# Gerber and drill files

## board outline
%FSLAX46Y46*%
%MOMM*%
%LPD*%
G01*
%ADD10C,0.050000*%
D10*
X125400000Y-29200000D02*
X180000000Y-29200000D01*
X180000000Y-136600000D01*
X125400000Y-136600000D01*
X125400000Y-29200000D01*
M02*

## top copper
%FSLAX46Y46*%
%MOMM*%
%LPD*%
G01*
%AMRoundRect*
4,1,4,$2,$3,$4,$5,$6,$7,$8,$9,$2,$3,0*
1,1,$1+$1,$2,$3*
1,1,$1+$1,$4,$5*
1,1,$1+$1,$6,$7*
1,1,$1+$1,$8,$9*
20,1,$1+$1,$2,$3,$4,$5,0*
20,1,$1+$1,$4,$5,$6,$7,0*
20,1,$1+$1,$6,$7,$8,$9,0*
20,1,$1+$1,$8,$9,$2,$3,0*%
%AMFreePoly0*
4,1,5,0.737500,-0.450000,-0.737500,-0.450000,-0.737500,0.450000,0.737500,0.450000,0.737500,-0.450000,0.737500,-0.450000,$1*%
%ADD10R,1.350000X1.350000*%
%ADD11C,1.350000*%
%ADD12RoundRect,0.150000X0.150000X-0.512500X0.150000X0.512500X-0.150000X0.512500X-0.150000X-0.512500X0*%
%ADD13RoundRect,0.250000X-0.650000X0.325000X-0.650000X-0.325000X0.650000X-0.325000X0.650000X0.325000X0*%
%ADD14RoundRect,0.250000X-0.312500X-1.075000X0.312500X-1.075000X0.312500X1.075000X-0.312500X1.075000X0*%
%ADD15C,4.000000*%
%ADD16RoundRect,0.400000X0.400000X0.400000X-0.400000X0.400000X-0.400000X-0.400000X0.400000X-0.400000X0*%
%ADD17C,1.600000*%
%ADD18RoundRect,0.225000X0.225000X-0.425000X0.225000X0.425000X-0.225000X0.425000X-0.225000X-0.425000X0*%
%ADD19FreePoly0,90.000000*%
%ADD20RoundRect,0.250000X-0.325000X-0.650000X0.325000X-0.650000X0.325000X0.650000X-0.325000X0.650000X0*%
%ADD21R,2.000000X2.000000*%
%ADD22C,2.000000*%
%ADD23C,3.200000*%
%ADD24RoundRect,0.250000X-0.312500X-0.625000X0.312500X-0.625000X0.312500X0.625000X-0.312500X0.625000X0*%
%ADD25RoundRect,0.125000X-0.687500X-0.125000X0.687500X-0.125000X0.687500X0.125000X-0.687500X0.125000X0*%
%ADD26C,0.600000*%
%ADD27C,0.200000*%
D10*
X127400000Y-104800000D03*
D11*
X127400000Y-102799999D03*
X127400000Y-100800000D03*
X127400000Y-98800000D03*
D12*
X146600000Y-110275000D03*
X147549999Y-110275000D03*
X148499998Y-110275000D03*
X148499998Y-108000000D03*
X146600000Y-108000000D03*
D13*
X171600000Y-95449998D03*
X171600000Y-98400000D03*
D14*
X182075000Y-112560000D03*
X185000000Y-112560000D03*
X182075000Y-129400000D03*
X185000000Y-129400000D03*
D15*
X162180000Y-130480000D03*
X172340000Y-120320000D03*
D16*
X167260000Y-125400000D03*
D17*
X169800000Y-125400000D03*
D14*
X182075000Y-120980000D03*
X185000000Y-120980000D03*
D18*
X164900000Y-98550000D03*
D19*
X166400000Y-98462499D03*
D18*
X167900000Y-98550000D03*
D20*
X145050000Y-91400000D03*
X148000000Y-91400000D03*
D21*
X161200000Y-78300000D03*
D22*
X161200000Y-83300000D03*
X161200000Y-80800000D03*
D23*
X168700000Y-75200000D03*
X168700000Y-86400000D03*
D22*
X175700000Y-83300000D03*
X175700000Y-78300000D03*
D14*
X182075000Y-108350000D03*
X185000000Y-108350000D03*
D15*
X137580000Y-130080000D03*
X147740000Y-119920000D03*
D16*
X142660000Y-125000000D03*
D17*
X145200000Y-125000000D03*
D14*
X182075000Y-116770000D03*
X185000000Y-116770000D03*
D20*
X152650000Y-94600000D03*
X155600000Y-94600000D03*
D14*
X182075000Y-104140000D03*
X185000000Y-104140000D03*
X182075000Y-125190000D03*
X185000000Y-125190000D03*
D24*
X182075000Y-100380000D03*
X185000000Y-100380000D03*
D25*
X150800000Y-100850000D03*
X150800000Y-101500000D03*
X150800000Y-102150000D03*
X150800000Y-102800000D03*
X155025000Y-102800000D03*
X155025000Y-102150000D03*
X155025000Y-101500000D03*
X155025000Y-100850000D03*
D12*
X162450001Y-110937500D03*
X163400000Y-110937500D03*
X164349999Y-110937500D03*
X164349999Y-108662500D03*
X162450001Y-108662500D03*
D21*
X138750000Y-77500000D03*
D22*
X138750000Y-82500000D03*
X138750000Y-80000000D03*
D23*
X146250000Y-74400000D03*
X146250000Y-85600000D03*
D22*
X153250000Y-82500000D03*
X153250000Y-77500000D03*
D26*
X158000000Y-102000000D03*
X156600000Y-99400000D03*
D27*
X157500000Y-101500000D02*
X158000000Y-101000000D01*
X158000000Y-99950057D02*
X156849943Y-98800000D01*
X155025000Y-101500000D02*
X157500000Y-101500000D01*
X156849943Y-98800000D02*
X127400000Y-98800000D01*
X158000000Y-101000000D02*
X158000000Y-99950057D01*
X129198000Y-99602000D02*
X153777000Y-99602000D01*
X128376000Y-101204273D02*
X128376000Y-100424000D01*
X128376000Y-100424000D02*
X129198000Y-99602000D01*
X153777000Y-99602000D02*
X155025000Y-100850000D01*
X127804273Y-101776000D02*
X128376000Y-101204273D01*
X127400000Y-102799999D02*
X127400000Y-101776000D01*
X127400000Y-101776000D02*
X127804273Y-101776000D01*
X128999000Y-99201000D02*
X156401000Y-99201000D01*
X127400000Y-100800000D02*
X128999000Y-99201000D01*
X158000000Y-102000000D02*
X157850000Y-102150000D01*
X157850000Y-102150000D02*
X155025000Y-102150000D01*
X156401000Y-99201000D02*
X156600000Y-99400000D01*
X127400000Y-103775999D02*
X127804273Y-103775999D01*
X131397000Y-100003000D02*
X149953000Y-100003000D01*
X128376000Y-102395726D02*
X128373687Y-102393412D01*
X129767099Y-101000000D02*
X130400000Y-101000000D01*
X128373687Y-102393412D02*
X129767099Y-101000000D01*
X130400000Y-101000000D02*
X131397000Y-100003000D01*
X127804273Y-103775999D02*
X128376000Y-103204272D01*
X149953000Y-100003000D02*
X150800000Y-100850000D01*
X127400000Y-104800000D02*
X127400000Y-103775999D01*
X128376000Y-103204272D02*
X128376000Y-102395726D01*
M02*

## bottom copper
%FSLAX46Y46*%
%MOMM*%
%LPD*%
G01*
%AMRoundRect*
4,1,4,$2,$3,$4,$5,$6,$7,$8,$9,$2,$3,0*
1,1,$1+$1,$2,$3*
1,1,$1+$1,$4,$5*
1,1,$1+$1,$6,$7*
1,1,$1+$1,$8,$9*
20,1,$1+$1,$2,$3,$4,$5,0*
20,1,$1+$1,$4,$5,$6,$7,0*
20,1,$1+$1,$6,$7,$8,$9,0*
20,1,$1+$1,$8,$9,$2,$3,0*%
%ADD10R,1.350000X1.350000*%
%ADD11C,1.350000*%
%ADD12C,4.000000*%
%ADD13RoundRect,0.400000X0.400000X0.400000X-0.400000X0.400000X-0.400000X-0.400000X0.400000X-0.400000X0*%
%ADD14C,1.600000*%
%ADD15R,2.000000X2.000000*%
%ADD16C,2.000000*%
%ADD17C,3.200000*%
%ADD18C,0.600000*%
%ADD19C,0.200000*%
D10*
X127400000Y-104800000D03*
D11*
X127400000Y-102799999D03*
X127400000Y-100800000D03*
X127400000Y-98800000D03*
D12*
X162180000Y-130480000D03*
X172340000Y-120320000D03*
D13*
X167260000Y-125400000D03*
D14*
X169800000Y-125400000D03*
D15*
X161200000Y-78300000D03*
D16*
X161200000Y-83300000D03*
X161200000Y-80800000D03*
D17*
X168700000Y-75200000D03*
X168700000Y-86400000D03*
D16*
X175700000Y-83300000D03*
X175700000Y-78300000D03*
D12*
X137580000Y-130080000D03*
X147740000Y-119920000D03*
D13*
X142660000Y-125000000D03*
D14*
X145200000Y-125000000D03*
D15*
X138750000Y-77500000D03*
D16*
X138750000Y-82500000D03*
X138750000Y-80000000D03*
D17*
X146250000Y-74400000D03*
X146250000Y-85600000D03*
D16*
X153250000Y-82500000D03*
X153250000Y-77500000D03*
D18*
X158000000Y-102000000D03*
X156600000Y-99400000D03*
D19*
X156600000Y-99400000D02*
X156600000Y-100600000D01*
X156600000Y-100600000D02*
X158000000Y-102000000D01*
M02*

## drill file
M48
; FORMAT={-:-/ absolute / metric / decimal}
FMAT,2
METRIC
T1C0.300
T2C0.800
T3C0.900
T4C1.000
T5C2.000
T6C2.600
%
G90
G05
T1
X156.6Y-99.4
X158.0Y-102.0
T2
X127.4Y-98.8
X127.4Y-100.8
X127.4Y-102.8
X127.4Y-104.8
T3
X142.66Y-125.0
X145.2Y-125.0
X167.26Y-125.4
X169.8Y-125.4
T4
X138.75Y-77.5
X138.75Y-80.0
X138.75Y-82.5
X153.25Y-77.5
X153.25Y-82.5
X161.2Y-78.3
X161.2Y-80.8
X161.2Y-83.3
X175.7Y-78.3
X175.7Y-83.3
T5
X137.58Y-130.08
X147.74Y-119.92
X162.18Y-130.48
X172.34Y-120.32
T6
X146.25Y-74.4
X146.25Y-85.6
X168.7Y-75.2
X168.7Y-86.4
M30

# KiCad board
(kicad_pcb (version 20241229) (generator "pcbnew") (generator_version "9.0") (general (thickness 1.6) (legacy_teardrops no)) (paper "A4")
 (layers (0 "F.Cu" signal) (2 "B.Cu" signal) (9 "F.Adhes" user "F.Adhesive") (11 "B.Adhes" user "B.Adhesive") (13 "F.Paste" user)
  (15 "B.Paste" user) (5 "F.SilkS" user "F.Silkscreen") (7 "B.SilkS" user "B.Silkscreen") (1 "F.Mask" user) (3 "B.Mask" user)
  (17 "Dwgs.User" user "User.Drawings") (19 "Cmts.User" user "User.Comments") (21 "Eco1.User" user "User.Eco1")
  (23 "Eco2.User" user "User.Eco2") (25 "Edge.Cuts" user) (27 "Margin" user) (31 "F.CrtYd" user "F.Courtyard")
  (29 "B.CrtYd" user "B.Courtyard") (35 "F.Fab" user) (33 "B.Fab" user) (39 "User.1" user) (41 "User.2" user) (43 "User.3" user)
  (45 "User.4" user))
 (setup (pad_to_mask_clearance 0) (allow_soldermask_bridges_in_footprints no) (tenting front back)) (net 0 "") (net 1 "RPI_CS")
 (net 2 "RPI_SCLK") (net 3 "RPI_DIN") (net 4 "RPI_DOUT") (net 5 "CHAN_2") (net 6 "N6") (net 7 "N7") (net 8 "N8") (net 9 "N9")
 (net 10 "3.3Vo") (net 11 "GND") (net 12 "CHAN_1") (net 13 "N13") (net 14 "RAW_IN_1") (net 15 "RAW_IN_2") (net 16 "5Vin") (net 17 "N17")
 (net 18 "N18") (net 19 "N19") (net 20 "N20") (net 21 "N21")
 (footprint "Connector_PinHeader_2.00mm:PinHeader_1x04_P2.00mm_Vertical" (layer "F.Cu") (at 127.4 104.8 180)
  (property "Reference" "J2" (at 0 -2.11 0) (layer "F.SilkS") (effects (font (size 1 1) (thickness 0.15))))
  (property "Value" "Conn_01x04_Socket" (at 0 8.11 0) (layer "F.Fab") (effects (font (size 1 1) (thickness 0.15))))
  (pad "1" thru_hole rect (at 0 0 180) (size 1.35 1.35) (drill 0.8) (layers "*.Cu" "*.Mask") (remove_unused_layers no) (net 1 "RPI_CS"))
  (pad "2" thru_hole circle (at 0 2.000001 180) (size 1.35 1.35) (drill 0.8) (layers "*.Cu" "*.Mask") (remove_unused_layers no)
   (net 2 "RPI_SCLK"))
  (pad "3" thru_hole circle (at 0 4 180) (size 1.35 1.35) (drill 0.8) (layers "*.Cu" "*.Mask") (remove_unused_layers no) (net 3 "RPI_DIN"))
  (pad "4" thru_hole circle (at 0 6 180) (size 1.35 1.35) (drill 0.8) (layers "*.Cu" "*.Mask") (remove_unused_layers no) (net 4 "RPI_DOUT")))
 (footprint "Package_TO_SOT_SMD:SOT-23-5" (layer "F.Cu") (at 147.549999 109.1375 90)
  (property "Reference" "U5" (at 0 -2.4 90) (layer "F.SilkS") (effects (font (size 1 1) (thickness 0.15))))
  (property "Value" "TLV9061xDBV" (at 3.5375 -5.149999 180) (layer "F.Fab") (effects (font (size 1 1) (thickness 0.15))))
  (pad "1" smd roundrect (at -1.1375 -0.949999 90) (size 1.325 0.6) (layers "F.Cu" "F.Mask" "F.Paste") (roundrect_rratio 0.25)
   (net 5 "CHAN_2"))
  (pad "2" smd roundrect (at -1.1375 0 90) (size 1.325 0.6) (layers "F.Cu" "F.Mask" "F.Paste") (roundrect_rratio 0.25) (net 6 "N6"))
  (pad "3" smd roundrect (at -1.1375 0.949999 90) (size 1.325 0.6) (layers "F.Cu" "F.Mask" "F.Paste") (roundrect_rratio 0.25) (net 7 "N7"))
  (pad "4" smd roundrect (at 1.1375 0.949999 90) (size 1.325 0.6) (layers "F.Cu" "F.Mask" "F.Paste") (roundrect_rratio 0.25) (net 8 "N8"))
  (pad "5" smd roundrect (at 1.1375 -0.949999 90) (size 1.325 0.6) (layers "F.Cu" "F.Mask" "F.Paste") (roundrect_rratio 0.25) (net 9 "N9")))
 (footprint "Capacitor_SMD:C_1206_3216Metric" (layer "F.Cu") (at 171.6 96.924999 -90)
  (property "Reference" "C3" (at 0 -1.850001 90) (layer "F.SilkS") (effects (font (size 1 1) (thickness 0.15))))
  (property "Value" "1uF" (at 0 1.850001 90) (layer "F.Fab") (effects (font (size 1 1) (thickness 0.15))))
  (pad "1" smd roundrect (at -1.475001 0 270) (size 1.15 1.8) (layers "F.Cu" "F.Mask" "F.Paste") (roundrect_rratio 0.217391)
   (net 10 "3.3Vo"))
  (pad "2" smd roundrect (at 1.475001 0 270) (size 1.15 1.8) (layers "F.Cu" "F.Mask" "F.Paste") (roundrect_rratio 0.217391) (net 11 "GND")))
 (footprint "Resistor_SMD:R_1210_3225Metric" (layer "F.Cu") (at 183.5375 112.56)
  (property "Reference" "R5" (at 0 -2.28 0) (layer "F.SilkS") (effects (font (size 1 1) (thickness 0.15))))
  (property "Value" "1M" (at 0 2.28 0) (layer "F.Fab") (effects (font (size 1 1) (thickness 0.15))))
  (pad "1" smd roundrect (at -1.4625 0) (size 1.125 2.65) (layers "F.Cu" "F.Mask" "F.Paste") (roundrect_rratio 0.222222) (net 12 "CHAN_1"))
  (pad "2" smd roundrect (at 1.4625 0) (size 1.125 2.65) (layers "F.Cu" "F.Mask" "F.Paste") (roundrect_rratio 0.222222) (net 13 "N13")))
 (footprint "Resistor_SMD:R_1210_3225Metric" (layer "F.Cu") (at 183.5375 129.4)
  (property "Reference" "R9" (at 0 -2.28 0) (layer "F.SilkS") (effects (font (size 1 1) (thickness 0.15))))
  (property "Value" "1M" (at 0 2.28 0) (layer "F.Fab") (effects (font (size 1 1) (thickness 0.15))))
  (pad "1" smd roundrect (at -1.4625 0) (size 1.125 2.65) (layers "F.Cu" "F.Mask" "F.Paste") (roundrect_rratio 0.222222) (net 5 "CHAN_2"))
  (pad "2" smd roundrect (at 1.4625 0) (size 1.125 2.65) (layers "F.Cu" "F.Mask" "F.Paste") (roundrect_rratio 0.222222) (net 8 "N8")))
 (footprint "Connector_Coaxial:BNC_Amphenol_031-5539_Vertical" (layer "F.Cu") (at 167.26 125.4)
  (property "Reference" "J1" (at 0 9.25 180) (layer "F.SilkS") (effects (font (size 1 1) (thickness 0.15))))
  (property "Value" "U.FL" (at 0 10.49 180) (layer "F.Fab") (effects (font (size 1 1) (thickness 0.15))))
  (pad "" thru_hole circle (at -5.08 5.08 180) (size 4 4) (drill 2) (layers "*.Cu" "*.Mask") (remove_unused_layers no))
  (pad "" thru_hole circle (at 5.08 -5.08 180) (size 4 4) (drill 2) (layers "*.Cu" "*.Mask") (remove_unused_layers no))
  (pad "1" thru_hole roundrect (at 0 0 180) (size 1.6 1.6) (drill 0.9) (layers "*.Cu" "*.Mask") (remove_unused_layers no)
   (roundrect_rratio 0.25) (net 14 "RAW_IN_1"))
  (pad "2" thru_hole circle (at 2.54 0 180) (size 1.6 1.6) (drill 0.9) (layers "*.Cu" "*.Mask") (remove_unused_layers no) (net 11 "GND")))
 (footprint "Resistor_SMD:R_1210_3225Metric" (layer "F.Cu") (at 183.5375 120.98)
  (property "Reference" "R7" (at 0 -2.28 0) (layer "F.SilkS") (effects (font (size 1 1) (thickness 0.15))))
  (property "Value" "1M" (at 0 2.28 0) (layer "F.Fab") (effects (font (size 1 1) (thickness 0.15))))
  (pad "1" smd roundrect (at -1.4625 0) (size 1.125 2.65) (layers "F.Cu" "F.Mask" "F.Paste") (roundrect_rratio 0.222222) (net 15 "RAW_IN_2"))
  (pad "2" smd roundrect (at 1.4625 0) (size 1.125 2.65) (layers "F.Cu" "F.Mask" "F.Paste") (roundrect_rratio 0.222222) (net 8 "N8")))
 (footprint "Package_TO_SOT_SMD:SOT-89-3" (layer "F.Cu") (at 166.4 96.6 90)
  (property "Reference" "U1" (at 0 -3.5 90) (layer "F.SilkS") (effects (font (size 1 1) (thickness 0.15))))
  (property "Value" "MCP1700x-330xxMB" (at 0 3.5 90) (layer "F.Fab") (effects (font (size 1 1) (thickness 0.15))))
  (pad "1" smd roundrect (at -1.95 -1.5 90) (size 1.3 0.9) (layers "F.Cu" "F.Mask" "F.Paste") (roundrect_rratio 0.25) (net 11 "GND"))
  (pad "2" smd custom (at -1.862499 0 90) (size 1.475 0.9) (layers "F.Cu" "F.Mask" "F.Paste") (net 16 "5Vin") (zone_connect 2)
   (thermal_bridge_angle 45) (options (clearance outline) (anchor rect)) (primitives))
  (pad "3" smd roundrect (at -1.95 1.5 90) (size 1.3 0.9) (layers "F.Cu" "F.Mask" "F.Paste") (roundrect_rratio 0.25) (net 10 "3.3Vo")))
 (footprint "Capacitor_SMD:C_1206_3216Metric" (layer "F.Cu") (at 146.525 91.4)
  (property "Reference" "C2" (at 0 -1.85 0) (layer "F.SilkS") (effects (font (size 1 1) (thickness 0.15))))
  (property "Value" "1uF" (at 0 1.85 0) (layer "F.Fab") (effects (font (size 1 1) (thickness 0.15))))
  (pad "1" smd roundrect (at -1.475 0) (size 1.15 1.8) (layers "F.Cu" "F.Mask" "F.Paste") (roundrect_rratio 0.217391) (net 10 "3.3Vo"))
  (pad "2" smd roundrect (at 1.475 0) (size 1.15 1.8) (layers "F.Cu" "F.Mask" "F.Paste") (roundrect_rratio 0.217391) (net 11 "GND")))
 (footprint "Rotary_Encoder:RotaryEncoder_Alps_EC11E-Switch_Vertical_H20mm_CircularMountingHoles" (layer "F.Cu") (at 161.2 78.3)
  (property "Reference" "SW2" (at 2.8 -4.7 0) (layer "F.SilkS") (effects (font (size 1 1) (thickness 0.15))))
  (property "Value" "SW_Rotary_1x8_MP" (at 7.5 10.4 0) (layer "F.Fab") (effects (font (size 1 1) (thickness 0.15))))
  (pad "A" thru_hole rect (at 0 0) (size 2 2) (drill 1) (layers "*.Cu" "*.Mask") (remove_unused_layers no))
  (pad "B" thru_hole circle (at 0 5) (size 2 2) (drill 1) (layers "*.Cu" "*.Mask") (remove_unused_layers no))
  (pad "C" thru_hole circle (at 0 2.5) (size 2 2) (drill 1) (layers "*.Cu" "*.Mask") (remove_unused_layers no))
  (pad "MP" thru_hole circle (at 7.5 -3.1) (size 3.2 3.2) (drill 2.6) (layers "*.Cu" "*.Mask") (remove_unused_layers no) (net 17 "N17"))
  (pad "MP" thru_hole circle (at 7.5 8.1) (size 3.2 3.2) (drill 2.6) (layers "*.Cu" "*.Mask") (remove_unused_layers no) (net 17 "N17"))
  (pad "S1" thru_hole circle (at 14.5 5) (size 2 2) (drill 1) (layers "*.Cu" "*.Mask") (remove_unused_layers no))
  (pad "S2" thru_hole circle (at 14.5 0) (size 2 2) (drill 1) (layers "*.Cu" "*.Mask") (remove_unused_layers no)))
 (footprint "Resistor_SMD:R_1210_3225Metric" (layer "F.Cu") (at 183.5375 108.35)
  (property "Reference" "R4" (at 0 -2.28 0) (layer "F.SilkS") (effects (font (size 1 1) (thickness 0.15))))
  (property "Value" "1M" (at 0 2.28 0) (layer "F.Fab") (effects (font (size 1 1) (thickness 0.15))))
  (pad "1" smd roundrect (at -1.4625 0) (size 1.125 2.65) (layers "F.Cu" "F.Mask" "F.Paste") (roundrect_rratio 0.222222) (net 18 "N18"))
  (pad "2" smd roundrect (at 1.4625 0) (size 1.125 2.65) (layers "F.Cu" "F.Mask" "F.Paste") (roundrect_rratio 0.222222) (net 11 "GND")))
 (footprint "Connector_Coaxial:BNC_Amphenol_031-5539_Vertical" (layer "F.Cu") (at 142.66 125)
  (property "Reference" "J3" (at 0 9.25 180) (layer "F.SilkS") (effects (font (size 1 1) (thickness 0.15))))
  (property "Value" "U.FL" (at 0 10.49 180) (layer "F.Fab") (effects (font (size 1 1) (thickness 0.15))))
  (pad "" thru_hole circle (at -5.08 5.08 180) (size 4 4) (drill 2) (layers "*.Cu" "*.Mask") (remove_unused_layers no))
  (pad "" thru_hole circle (at 5.08 -5.08 180) (size 4 4) (drill 2) (layers "*.Cu" "*.Mask") (remove_unused_layers no))
  (pad "1" thru_hole roundrect (at 0 0 180) (size 1.6 1.6) (drill 0.9) (layers "*.Cu" "*.Mask") (remove_unused_layers no)
   (roundrect_rratio 0.25) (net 15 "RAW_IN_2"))
  (pad "2" thru_hole circle (at 2.54 0 180) (size 1.6 1.6) (drill 0.9) (layers "*.Cu" "*.Mask") (remove_unused_layers no) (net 11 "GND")))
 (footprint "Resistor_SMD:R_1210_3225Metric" (layer "F.Cu") (at 183.5375 116.77)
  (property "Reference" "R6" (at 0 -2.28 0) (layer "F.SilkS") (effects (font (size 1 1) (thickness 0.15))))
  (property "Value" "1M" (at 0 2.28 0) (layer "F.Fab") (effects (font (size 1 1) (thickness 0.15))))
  (pad "1" smd roundrect (at -1.4625 0) (size 1.125 2.65) (layers "F.Cu" "F.Mask" "F.Paste") (roundrect_rratio 0.222222) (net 14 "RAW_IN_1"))
  (pad "2" smd roundrect (at 1.4625 0) (size 1.125 2.65) (layers "F.Cu" "F.Mask" "F.Paste") (roundrect_rratio 0.222222) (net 13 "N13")))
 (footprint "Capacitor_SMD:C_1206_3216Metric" (layer "F.Cu") (at 154.125 94.6)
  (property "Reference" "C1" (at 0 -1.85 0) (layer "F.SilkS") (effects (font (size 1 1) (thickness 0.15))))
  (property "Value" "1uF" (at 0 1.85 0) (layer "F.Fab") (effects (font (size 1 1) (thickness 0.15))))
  (pad "1" smd roundrect (at -1.475 0) (size 1.15 1.8) (layers "F.Cu" "F.Mask" "F.Paste") (roundrect_rratio 0.217391) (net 16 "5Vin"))
  (pad "2" smd roundrect (at 1.475 0) (size 1.15 1.8) (layers "F.Cu" "F.Mask" "F.Paste") (roundrect_rratio 0.217391) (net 11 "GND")))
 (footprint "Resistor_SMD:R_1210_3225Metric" (layer "F.Cu") (at 183.5375 104.14)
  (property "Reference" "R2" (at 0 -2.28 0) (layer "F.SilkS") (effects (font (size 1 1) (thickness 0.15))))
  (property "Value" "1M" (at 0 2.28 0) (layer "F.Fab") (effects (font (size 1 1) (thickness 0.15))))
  (pad "1" smd roundrect (at -1.4625 0) (size 1.125 2.65) (layers "F.Cu" "F.Mask" "F.Paste") (roundrect_rratio 0.222222) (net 15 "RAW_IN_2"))
  (pad "2" smd roundrect (at 1.4625 0) (size 1.125 2.65) (layers "F.Cu" "F.Mask" "F.Paste") (roundrect_rratio 0.222222) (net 11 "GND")))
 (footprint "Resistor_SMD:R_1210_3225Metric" (layer "F.Cu") (at 183.5375 125.19)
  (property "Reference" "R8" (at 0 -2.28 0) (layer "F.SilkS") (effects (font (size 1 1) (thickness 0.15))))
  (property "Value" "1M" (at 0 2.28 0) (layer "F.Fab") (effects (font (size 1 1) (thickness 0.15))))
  (pad "1" smd roundrect (at -1.4625 0) (size 1.125 2.65) (layers "F.Cu" "F.Mask" "F.Paste") (roundrect_rratio 0.222222) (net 7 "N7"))
  (pad "2" smd roundrect (at 1.4625 0) (size 1.125 2.65) (layers "F.Cu" "F.Mask" "F.Paste") (roundrect_rratio 0.222222) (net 11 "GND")))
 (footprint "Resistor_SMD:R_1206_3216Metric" (layer "F.Cu") (at 183.5375 100.38)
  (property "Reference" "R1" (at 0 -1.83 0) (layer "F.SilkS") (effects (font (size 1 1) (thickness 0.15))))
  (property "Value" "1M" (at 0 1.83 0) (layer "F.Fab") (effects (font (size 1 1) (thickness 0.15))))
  (pad "1" smd roundrect (at -1.4625 0) (size 1.125 1.75) (layers "F.Cu" "F.Mask" "F.Paste") (roundrect_rratio 0.222222) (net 14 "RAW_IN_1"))
  (pad "2" smd roundrect (at 1.4625 0) (size 1.125 1.75) (layers "F.Cu" "F.Mask" "F.Paste") (roundrect_rratio 0.222222) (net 11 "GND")))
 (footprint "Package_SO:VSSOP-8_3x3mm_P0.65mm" (layer "F.Cu") (at 152.9125 101.825)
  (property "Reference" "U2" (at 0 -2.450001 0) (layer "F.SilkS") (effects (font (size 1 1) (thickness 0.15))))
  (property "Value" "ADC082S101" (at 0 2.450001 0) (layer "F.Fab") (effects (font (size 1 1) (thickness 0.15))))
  (pad "1" smd roundrect (at -2.1125 -0.975) (size 1.625 0.5) (layers "F.Cu" "F.Mask" "F.Paste") (roundrect_rratio 0.25) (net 1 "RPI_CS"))
  (pad "2" smd roundrect (at -2.1125 -0.325) (size 1.625 0.5) (layers "F.Cu" "F.Mask" "F.Paste") (roundrect_rratio 0.25) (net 10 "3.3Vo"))
  (pad "3" smd roundrect (at -2.1125 0.325) (size 1.625 0.5) (layers "F.Cu" "F.Mask" "F.Paste") (roundrect_rratio 0.25) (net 11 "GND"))
  (pad "4" smd roundrect (at -2.1125 0.975) (size 1.625 0.5) (layers "F.Cu" "F.Mask" "F.Paste") (roundrect_rratio 0.25) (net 5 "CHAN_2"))
  (pad "5" smd roundrect (at 2.1125 0.975) (size 1.625 0.5) (layers "F.Cu" "F.Mask" "F.Paste") (roundrect_rratio 0.25) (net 12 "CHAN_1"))
  (pad "6" smd roundrect (at 2.1125 0.325) (size 1.625 0.5) (layers "F.Cu" "F.Mask" "F.Paste") (roundrect_rratio 0.25) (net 3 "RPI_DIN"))
  (pad "7" smd roundrect (at 2.1125 -0.325) (size 1.625 0.5) (layers "F.Cu" "F.Mask" "F.Paste") (roundrect_rratio 0.25) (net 4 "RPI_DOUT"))
  (pad "8" smd roundrect (at 2.1125 -0.975) (size 1.625 0.5) (layers "F.Cu" "F.Mask" "F.Paste") (roundrect_rratio 0.25) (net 2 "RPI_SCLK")))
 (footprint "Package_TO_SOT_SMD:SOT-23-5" (layer "F.Cu") (at 163.4 109.8 90)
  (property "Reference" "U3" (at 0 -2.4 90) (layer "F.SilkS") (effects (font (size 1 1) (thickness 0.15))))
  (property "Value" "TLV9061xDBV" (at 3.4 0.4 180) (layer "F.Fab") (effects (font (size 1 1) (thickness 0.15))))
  (pad "1" smd roundrect (at -1.1375 -0.949999 90) (size 1.325 0.6) (layers "F.Cu" "F.Mask" "F.Paste") (roundrect_rratio 0.25)
   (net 12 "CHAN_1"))
  (pad "2" smd roundrect (at -1.1375 0 90) (size 1.325 0.6) (layers "F.Cu" "F.Mask" "F.Paste") (roundrect_rratio 0.25) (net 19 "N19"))
  (pad "3" smd roundrect (at -1.1375 0.949999 90) (size 1.325 0.6) (layers "F.Cu" "F.Mask" "F.Paste") (roundrect_rratio 0.25) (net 18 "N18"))
  (pad "4" smd roundrect (at 1.1375 0.949999 90) (size 1.325 0.6) (layers "F.Cu" "F.Mask" "F.Paste") (roundrect_rratio 0.25) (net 13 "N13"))
  (pad "5" smd roundrect (at 1.1375 -0.949999 90) (size 1.325 0.6) (layers "F.Cu" "F.Mask" "F.Paste") (roundrect_rratio 0.25) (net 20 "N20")))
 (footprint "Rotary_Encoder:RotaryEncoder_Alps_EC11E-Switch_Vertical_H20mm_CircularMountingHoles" (layer "F.Cu") (at 138.75 77.5)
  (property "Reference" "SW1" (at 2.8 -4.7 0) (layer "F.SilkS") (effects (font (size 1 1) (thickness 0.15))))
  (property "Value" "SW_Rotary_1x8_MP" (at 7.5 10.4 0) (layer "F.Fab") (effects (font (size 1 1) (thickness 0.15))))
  (pad "A" thru_hole rect (at 0 0) (size 2 2) (drill 1) (layers "*.Cu" "*.Mask") (remove_unused_layers no))
  (pad "B" thru_hole circle (at 0 5) (size 2 2) (drill 1) (layers "*.Cu" "*.Mask") (remove_unused_layers no))
  (pad "C" thru_hole circle (at 0 2.5) (size 2 2) (drill 1) (layers "*.Cu" "*.Mask") (remove_unused_layers no))
  (pad "MP" thru_hole circle (at 7.5 -3.1) (size 3.2 3.2) (drill 2.6) (layers "*.Cu" "*.Mask") (remove_unused_layers no) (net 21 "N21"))
  (pad "MP" thru_hole circle (at 7.5 8.1) (size 3.2 3.2) (drill 2.6) (layers "*.Cu" "*.Mask") (remove_unused_layers no) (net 21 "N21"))
  (pad "S1" thru_hole circle (at 14.5 5) (size 2 2) (drill 1) (layers "*.Cu" "*.Mask") (remove_unused_layers no))
  (pad "S2" thru_hole circle (at 14.5 0) (size 2 2) (drill 1) (layers "*.Cu" "*.Mask") (remove_unused_layers no)))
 (gr_rect (start 125.4 29.2) (end 180 136.6) (stroke (width 0.05) (type default)) (fill no) (layer "Edge.Cuts"))
 (segment (start 157.5 101.5) (end 158 101) (width 0.2) (layer "F.Cu") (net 4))
 (segment (start 158 99.950057) (end 156.849943 98.8) (width 0.2) (layer "F.Cu") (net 4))
 (segment (start 155.025 101.5) (end 157.5 101.5) (width 0.2) (layer "F.Cu") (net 4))
 (segment (start 156.849943 98.8) (end 127.4 98.8) (width 0.2) (layer "F.Cu") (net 4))
 (segment (start 158 101) (end 158 99.950057) (width 0.2) (layer "F.Cu") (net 4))
 (segment (start 129.198 99.602) (end 153.777 99.602) (width 0.2) (layer "F.Cu") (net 2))
 (segment (start 128.376 101.204273) (end 128.376 100.424) (width 0.2) (layer "F.Cu") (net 2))
 (segment (start 128.376 100.424) (end 129.198 99.602) (width 0.2) (layer "F.Cu") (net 2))
 (segment (start 153.777 99.602) (end 155.025 100.85) (width 0.2) (layer "F.Cu") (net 2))
 (segment (start 127.804273 101.776) (end 128.376 101.204273) (width 0.2) (layer "F.Cu") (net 2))
 (segment (start 127.4 102.799999) (end 127.4 101.776) (width 0.2) (layer "F.Cu") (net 2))
 (segment (start 127.4 101.776) (end 127.804273 101.776) (width 0.2) (layer "F.Cu") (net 2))
 (segment (start 128.999 99.201) (end 156.401 99.201) (width 0.2) (layer "F.Cu") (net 3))
 (segment (start 127.4 100.8) (end 128.999 99.201) (width 0.2) (layer "F.Cu") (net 3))
 (segment (start 158 102) (end 157.85 102.15) (width 0.2) (layer "F.Cu") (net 3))
 (segment (start 157.85 102.15) (end 155.025 102.15) (width 0.2) (layer "F.Cu") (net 3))
 (segment (start 156.401 99.201) (end 156.6 99.4) (width 0.2) (layer "F.Cu") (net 3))
 (via (at 158 102) (size 0.6) (drill 0.3) (layers "F.Cu" "B.Cu") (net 3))
 (via (at 156.6 99.4) (size 0.6) (drill 0.3) (layers "F.Cu" "B.Cu") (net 3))
 (segment (start 156.6 99.4) (end 156.6 100.6) (width 0.2) (layer "B.Cu") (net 3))
 (segment (start 156.6 100.6) (end 158 102) (width 0.2) (layer "B.Cu") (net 3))
 (segment (start 127.4 103.775999) (end 127.804273 103.775999) (width 0.2) (layer "F.Cu") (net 1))
 (segment (start 131.397 100.003) (end 149.953 100.003) (width 0.2) (layer "F.Cu") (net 1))
 (segment (start 128.376 102.395726) (end 128.373687 102.393412) (width 0.2) (layer "F.Cu") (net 1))
 (segment (start 129.767099 101) (end 130.4 101) (width 0.2) (layer "F.Cu") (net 1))
 (segment (start 128.373687 102.393412) (end 129.767099 101) (width 0.2) (layer "F.Cu") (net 1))
 (segment (start 130.4 101) (end 131.397 100.003) (width 0.2) (layer "F.Cu") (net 1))
 (segment (start 127.804273 103.775999) (end 128.376 103.204272) (width 0.2) (layer "F.Cu") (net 1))
 (segment (start 149.953 100.003) (end 150.8 100.85) (width 0.2) (layer "F.Cu") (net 1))
 (segment (start 127.4 104.8) (end 127.4 103.775999) (width 0.2) (layer "F.Cu") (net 1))
 (segment (start 128.376 103.204272) (end 128.376 102.395726) (width 0.2) (layer "F.Cu") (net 1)))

